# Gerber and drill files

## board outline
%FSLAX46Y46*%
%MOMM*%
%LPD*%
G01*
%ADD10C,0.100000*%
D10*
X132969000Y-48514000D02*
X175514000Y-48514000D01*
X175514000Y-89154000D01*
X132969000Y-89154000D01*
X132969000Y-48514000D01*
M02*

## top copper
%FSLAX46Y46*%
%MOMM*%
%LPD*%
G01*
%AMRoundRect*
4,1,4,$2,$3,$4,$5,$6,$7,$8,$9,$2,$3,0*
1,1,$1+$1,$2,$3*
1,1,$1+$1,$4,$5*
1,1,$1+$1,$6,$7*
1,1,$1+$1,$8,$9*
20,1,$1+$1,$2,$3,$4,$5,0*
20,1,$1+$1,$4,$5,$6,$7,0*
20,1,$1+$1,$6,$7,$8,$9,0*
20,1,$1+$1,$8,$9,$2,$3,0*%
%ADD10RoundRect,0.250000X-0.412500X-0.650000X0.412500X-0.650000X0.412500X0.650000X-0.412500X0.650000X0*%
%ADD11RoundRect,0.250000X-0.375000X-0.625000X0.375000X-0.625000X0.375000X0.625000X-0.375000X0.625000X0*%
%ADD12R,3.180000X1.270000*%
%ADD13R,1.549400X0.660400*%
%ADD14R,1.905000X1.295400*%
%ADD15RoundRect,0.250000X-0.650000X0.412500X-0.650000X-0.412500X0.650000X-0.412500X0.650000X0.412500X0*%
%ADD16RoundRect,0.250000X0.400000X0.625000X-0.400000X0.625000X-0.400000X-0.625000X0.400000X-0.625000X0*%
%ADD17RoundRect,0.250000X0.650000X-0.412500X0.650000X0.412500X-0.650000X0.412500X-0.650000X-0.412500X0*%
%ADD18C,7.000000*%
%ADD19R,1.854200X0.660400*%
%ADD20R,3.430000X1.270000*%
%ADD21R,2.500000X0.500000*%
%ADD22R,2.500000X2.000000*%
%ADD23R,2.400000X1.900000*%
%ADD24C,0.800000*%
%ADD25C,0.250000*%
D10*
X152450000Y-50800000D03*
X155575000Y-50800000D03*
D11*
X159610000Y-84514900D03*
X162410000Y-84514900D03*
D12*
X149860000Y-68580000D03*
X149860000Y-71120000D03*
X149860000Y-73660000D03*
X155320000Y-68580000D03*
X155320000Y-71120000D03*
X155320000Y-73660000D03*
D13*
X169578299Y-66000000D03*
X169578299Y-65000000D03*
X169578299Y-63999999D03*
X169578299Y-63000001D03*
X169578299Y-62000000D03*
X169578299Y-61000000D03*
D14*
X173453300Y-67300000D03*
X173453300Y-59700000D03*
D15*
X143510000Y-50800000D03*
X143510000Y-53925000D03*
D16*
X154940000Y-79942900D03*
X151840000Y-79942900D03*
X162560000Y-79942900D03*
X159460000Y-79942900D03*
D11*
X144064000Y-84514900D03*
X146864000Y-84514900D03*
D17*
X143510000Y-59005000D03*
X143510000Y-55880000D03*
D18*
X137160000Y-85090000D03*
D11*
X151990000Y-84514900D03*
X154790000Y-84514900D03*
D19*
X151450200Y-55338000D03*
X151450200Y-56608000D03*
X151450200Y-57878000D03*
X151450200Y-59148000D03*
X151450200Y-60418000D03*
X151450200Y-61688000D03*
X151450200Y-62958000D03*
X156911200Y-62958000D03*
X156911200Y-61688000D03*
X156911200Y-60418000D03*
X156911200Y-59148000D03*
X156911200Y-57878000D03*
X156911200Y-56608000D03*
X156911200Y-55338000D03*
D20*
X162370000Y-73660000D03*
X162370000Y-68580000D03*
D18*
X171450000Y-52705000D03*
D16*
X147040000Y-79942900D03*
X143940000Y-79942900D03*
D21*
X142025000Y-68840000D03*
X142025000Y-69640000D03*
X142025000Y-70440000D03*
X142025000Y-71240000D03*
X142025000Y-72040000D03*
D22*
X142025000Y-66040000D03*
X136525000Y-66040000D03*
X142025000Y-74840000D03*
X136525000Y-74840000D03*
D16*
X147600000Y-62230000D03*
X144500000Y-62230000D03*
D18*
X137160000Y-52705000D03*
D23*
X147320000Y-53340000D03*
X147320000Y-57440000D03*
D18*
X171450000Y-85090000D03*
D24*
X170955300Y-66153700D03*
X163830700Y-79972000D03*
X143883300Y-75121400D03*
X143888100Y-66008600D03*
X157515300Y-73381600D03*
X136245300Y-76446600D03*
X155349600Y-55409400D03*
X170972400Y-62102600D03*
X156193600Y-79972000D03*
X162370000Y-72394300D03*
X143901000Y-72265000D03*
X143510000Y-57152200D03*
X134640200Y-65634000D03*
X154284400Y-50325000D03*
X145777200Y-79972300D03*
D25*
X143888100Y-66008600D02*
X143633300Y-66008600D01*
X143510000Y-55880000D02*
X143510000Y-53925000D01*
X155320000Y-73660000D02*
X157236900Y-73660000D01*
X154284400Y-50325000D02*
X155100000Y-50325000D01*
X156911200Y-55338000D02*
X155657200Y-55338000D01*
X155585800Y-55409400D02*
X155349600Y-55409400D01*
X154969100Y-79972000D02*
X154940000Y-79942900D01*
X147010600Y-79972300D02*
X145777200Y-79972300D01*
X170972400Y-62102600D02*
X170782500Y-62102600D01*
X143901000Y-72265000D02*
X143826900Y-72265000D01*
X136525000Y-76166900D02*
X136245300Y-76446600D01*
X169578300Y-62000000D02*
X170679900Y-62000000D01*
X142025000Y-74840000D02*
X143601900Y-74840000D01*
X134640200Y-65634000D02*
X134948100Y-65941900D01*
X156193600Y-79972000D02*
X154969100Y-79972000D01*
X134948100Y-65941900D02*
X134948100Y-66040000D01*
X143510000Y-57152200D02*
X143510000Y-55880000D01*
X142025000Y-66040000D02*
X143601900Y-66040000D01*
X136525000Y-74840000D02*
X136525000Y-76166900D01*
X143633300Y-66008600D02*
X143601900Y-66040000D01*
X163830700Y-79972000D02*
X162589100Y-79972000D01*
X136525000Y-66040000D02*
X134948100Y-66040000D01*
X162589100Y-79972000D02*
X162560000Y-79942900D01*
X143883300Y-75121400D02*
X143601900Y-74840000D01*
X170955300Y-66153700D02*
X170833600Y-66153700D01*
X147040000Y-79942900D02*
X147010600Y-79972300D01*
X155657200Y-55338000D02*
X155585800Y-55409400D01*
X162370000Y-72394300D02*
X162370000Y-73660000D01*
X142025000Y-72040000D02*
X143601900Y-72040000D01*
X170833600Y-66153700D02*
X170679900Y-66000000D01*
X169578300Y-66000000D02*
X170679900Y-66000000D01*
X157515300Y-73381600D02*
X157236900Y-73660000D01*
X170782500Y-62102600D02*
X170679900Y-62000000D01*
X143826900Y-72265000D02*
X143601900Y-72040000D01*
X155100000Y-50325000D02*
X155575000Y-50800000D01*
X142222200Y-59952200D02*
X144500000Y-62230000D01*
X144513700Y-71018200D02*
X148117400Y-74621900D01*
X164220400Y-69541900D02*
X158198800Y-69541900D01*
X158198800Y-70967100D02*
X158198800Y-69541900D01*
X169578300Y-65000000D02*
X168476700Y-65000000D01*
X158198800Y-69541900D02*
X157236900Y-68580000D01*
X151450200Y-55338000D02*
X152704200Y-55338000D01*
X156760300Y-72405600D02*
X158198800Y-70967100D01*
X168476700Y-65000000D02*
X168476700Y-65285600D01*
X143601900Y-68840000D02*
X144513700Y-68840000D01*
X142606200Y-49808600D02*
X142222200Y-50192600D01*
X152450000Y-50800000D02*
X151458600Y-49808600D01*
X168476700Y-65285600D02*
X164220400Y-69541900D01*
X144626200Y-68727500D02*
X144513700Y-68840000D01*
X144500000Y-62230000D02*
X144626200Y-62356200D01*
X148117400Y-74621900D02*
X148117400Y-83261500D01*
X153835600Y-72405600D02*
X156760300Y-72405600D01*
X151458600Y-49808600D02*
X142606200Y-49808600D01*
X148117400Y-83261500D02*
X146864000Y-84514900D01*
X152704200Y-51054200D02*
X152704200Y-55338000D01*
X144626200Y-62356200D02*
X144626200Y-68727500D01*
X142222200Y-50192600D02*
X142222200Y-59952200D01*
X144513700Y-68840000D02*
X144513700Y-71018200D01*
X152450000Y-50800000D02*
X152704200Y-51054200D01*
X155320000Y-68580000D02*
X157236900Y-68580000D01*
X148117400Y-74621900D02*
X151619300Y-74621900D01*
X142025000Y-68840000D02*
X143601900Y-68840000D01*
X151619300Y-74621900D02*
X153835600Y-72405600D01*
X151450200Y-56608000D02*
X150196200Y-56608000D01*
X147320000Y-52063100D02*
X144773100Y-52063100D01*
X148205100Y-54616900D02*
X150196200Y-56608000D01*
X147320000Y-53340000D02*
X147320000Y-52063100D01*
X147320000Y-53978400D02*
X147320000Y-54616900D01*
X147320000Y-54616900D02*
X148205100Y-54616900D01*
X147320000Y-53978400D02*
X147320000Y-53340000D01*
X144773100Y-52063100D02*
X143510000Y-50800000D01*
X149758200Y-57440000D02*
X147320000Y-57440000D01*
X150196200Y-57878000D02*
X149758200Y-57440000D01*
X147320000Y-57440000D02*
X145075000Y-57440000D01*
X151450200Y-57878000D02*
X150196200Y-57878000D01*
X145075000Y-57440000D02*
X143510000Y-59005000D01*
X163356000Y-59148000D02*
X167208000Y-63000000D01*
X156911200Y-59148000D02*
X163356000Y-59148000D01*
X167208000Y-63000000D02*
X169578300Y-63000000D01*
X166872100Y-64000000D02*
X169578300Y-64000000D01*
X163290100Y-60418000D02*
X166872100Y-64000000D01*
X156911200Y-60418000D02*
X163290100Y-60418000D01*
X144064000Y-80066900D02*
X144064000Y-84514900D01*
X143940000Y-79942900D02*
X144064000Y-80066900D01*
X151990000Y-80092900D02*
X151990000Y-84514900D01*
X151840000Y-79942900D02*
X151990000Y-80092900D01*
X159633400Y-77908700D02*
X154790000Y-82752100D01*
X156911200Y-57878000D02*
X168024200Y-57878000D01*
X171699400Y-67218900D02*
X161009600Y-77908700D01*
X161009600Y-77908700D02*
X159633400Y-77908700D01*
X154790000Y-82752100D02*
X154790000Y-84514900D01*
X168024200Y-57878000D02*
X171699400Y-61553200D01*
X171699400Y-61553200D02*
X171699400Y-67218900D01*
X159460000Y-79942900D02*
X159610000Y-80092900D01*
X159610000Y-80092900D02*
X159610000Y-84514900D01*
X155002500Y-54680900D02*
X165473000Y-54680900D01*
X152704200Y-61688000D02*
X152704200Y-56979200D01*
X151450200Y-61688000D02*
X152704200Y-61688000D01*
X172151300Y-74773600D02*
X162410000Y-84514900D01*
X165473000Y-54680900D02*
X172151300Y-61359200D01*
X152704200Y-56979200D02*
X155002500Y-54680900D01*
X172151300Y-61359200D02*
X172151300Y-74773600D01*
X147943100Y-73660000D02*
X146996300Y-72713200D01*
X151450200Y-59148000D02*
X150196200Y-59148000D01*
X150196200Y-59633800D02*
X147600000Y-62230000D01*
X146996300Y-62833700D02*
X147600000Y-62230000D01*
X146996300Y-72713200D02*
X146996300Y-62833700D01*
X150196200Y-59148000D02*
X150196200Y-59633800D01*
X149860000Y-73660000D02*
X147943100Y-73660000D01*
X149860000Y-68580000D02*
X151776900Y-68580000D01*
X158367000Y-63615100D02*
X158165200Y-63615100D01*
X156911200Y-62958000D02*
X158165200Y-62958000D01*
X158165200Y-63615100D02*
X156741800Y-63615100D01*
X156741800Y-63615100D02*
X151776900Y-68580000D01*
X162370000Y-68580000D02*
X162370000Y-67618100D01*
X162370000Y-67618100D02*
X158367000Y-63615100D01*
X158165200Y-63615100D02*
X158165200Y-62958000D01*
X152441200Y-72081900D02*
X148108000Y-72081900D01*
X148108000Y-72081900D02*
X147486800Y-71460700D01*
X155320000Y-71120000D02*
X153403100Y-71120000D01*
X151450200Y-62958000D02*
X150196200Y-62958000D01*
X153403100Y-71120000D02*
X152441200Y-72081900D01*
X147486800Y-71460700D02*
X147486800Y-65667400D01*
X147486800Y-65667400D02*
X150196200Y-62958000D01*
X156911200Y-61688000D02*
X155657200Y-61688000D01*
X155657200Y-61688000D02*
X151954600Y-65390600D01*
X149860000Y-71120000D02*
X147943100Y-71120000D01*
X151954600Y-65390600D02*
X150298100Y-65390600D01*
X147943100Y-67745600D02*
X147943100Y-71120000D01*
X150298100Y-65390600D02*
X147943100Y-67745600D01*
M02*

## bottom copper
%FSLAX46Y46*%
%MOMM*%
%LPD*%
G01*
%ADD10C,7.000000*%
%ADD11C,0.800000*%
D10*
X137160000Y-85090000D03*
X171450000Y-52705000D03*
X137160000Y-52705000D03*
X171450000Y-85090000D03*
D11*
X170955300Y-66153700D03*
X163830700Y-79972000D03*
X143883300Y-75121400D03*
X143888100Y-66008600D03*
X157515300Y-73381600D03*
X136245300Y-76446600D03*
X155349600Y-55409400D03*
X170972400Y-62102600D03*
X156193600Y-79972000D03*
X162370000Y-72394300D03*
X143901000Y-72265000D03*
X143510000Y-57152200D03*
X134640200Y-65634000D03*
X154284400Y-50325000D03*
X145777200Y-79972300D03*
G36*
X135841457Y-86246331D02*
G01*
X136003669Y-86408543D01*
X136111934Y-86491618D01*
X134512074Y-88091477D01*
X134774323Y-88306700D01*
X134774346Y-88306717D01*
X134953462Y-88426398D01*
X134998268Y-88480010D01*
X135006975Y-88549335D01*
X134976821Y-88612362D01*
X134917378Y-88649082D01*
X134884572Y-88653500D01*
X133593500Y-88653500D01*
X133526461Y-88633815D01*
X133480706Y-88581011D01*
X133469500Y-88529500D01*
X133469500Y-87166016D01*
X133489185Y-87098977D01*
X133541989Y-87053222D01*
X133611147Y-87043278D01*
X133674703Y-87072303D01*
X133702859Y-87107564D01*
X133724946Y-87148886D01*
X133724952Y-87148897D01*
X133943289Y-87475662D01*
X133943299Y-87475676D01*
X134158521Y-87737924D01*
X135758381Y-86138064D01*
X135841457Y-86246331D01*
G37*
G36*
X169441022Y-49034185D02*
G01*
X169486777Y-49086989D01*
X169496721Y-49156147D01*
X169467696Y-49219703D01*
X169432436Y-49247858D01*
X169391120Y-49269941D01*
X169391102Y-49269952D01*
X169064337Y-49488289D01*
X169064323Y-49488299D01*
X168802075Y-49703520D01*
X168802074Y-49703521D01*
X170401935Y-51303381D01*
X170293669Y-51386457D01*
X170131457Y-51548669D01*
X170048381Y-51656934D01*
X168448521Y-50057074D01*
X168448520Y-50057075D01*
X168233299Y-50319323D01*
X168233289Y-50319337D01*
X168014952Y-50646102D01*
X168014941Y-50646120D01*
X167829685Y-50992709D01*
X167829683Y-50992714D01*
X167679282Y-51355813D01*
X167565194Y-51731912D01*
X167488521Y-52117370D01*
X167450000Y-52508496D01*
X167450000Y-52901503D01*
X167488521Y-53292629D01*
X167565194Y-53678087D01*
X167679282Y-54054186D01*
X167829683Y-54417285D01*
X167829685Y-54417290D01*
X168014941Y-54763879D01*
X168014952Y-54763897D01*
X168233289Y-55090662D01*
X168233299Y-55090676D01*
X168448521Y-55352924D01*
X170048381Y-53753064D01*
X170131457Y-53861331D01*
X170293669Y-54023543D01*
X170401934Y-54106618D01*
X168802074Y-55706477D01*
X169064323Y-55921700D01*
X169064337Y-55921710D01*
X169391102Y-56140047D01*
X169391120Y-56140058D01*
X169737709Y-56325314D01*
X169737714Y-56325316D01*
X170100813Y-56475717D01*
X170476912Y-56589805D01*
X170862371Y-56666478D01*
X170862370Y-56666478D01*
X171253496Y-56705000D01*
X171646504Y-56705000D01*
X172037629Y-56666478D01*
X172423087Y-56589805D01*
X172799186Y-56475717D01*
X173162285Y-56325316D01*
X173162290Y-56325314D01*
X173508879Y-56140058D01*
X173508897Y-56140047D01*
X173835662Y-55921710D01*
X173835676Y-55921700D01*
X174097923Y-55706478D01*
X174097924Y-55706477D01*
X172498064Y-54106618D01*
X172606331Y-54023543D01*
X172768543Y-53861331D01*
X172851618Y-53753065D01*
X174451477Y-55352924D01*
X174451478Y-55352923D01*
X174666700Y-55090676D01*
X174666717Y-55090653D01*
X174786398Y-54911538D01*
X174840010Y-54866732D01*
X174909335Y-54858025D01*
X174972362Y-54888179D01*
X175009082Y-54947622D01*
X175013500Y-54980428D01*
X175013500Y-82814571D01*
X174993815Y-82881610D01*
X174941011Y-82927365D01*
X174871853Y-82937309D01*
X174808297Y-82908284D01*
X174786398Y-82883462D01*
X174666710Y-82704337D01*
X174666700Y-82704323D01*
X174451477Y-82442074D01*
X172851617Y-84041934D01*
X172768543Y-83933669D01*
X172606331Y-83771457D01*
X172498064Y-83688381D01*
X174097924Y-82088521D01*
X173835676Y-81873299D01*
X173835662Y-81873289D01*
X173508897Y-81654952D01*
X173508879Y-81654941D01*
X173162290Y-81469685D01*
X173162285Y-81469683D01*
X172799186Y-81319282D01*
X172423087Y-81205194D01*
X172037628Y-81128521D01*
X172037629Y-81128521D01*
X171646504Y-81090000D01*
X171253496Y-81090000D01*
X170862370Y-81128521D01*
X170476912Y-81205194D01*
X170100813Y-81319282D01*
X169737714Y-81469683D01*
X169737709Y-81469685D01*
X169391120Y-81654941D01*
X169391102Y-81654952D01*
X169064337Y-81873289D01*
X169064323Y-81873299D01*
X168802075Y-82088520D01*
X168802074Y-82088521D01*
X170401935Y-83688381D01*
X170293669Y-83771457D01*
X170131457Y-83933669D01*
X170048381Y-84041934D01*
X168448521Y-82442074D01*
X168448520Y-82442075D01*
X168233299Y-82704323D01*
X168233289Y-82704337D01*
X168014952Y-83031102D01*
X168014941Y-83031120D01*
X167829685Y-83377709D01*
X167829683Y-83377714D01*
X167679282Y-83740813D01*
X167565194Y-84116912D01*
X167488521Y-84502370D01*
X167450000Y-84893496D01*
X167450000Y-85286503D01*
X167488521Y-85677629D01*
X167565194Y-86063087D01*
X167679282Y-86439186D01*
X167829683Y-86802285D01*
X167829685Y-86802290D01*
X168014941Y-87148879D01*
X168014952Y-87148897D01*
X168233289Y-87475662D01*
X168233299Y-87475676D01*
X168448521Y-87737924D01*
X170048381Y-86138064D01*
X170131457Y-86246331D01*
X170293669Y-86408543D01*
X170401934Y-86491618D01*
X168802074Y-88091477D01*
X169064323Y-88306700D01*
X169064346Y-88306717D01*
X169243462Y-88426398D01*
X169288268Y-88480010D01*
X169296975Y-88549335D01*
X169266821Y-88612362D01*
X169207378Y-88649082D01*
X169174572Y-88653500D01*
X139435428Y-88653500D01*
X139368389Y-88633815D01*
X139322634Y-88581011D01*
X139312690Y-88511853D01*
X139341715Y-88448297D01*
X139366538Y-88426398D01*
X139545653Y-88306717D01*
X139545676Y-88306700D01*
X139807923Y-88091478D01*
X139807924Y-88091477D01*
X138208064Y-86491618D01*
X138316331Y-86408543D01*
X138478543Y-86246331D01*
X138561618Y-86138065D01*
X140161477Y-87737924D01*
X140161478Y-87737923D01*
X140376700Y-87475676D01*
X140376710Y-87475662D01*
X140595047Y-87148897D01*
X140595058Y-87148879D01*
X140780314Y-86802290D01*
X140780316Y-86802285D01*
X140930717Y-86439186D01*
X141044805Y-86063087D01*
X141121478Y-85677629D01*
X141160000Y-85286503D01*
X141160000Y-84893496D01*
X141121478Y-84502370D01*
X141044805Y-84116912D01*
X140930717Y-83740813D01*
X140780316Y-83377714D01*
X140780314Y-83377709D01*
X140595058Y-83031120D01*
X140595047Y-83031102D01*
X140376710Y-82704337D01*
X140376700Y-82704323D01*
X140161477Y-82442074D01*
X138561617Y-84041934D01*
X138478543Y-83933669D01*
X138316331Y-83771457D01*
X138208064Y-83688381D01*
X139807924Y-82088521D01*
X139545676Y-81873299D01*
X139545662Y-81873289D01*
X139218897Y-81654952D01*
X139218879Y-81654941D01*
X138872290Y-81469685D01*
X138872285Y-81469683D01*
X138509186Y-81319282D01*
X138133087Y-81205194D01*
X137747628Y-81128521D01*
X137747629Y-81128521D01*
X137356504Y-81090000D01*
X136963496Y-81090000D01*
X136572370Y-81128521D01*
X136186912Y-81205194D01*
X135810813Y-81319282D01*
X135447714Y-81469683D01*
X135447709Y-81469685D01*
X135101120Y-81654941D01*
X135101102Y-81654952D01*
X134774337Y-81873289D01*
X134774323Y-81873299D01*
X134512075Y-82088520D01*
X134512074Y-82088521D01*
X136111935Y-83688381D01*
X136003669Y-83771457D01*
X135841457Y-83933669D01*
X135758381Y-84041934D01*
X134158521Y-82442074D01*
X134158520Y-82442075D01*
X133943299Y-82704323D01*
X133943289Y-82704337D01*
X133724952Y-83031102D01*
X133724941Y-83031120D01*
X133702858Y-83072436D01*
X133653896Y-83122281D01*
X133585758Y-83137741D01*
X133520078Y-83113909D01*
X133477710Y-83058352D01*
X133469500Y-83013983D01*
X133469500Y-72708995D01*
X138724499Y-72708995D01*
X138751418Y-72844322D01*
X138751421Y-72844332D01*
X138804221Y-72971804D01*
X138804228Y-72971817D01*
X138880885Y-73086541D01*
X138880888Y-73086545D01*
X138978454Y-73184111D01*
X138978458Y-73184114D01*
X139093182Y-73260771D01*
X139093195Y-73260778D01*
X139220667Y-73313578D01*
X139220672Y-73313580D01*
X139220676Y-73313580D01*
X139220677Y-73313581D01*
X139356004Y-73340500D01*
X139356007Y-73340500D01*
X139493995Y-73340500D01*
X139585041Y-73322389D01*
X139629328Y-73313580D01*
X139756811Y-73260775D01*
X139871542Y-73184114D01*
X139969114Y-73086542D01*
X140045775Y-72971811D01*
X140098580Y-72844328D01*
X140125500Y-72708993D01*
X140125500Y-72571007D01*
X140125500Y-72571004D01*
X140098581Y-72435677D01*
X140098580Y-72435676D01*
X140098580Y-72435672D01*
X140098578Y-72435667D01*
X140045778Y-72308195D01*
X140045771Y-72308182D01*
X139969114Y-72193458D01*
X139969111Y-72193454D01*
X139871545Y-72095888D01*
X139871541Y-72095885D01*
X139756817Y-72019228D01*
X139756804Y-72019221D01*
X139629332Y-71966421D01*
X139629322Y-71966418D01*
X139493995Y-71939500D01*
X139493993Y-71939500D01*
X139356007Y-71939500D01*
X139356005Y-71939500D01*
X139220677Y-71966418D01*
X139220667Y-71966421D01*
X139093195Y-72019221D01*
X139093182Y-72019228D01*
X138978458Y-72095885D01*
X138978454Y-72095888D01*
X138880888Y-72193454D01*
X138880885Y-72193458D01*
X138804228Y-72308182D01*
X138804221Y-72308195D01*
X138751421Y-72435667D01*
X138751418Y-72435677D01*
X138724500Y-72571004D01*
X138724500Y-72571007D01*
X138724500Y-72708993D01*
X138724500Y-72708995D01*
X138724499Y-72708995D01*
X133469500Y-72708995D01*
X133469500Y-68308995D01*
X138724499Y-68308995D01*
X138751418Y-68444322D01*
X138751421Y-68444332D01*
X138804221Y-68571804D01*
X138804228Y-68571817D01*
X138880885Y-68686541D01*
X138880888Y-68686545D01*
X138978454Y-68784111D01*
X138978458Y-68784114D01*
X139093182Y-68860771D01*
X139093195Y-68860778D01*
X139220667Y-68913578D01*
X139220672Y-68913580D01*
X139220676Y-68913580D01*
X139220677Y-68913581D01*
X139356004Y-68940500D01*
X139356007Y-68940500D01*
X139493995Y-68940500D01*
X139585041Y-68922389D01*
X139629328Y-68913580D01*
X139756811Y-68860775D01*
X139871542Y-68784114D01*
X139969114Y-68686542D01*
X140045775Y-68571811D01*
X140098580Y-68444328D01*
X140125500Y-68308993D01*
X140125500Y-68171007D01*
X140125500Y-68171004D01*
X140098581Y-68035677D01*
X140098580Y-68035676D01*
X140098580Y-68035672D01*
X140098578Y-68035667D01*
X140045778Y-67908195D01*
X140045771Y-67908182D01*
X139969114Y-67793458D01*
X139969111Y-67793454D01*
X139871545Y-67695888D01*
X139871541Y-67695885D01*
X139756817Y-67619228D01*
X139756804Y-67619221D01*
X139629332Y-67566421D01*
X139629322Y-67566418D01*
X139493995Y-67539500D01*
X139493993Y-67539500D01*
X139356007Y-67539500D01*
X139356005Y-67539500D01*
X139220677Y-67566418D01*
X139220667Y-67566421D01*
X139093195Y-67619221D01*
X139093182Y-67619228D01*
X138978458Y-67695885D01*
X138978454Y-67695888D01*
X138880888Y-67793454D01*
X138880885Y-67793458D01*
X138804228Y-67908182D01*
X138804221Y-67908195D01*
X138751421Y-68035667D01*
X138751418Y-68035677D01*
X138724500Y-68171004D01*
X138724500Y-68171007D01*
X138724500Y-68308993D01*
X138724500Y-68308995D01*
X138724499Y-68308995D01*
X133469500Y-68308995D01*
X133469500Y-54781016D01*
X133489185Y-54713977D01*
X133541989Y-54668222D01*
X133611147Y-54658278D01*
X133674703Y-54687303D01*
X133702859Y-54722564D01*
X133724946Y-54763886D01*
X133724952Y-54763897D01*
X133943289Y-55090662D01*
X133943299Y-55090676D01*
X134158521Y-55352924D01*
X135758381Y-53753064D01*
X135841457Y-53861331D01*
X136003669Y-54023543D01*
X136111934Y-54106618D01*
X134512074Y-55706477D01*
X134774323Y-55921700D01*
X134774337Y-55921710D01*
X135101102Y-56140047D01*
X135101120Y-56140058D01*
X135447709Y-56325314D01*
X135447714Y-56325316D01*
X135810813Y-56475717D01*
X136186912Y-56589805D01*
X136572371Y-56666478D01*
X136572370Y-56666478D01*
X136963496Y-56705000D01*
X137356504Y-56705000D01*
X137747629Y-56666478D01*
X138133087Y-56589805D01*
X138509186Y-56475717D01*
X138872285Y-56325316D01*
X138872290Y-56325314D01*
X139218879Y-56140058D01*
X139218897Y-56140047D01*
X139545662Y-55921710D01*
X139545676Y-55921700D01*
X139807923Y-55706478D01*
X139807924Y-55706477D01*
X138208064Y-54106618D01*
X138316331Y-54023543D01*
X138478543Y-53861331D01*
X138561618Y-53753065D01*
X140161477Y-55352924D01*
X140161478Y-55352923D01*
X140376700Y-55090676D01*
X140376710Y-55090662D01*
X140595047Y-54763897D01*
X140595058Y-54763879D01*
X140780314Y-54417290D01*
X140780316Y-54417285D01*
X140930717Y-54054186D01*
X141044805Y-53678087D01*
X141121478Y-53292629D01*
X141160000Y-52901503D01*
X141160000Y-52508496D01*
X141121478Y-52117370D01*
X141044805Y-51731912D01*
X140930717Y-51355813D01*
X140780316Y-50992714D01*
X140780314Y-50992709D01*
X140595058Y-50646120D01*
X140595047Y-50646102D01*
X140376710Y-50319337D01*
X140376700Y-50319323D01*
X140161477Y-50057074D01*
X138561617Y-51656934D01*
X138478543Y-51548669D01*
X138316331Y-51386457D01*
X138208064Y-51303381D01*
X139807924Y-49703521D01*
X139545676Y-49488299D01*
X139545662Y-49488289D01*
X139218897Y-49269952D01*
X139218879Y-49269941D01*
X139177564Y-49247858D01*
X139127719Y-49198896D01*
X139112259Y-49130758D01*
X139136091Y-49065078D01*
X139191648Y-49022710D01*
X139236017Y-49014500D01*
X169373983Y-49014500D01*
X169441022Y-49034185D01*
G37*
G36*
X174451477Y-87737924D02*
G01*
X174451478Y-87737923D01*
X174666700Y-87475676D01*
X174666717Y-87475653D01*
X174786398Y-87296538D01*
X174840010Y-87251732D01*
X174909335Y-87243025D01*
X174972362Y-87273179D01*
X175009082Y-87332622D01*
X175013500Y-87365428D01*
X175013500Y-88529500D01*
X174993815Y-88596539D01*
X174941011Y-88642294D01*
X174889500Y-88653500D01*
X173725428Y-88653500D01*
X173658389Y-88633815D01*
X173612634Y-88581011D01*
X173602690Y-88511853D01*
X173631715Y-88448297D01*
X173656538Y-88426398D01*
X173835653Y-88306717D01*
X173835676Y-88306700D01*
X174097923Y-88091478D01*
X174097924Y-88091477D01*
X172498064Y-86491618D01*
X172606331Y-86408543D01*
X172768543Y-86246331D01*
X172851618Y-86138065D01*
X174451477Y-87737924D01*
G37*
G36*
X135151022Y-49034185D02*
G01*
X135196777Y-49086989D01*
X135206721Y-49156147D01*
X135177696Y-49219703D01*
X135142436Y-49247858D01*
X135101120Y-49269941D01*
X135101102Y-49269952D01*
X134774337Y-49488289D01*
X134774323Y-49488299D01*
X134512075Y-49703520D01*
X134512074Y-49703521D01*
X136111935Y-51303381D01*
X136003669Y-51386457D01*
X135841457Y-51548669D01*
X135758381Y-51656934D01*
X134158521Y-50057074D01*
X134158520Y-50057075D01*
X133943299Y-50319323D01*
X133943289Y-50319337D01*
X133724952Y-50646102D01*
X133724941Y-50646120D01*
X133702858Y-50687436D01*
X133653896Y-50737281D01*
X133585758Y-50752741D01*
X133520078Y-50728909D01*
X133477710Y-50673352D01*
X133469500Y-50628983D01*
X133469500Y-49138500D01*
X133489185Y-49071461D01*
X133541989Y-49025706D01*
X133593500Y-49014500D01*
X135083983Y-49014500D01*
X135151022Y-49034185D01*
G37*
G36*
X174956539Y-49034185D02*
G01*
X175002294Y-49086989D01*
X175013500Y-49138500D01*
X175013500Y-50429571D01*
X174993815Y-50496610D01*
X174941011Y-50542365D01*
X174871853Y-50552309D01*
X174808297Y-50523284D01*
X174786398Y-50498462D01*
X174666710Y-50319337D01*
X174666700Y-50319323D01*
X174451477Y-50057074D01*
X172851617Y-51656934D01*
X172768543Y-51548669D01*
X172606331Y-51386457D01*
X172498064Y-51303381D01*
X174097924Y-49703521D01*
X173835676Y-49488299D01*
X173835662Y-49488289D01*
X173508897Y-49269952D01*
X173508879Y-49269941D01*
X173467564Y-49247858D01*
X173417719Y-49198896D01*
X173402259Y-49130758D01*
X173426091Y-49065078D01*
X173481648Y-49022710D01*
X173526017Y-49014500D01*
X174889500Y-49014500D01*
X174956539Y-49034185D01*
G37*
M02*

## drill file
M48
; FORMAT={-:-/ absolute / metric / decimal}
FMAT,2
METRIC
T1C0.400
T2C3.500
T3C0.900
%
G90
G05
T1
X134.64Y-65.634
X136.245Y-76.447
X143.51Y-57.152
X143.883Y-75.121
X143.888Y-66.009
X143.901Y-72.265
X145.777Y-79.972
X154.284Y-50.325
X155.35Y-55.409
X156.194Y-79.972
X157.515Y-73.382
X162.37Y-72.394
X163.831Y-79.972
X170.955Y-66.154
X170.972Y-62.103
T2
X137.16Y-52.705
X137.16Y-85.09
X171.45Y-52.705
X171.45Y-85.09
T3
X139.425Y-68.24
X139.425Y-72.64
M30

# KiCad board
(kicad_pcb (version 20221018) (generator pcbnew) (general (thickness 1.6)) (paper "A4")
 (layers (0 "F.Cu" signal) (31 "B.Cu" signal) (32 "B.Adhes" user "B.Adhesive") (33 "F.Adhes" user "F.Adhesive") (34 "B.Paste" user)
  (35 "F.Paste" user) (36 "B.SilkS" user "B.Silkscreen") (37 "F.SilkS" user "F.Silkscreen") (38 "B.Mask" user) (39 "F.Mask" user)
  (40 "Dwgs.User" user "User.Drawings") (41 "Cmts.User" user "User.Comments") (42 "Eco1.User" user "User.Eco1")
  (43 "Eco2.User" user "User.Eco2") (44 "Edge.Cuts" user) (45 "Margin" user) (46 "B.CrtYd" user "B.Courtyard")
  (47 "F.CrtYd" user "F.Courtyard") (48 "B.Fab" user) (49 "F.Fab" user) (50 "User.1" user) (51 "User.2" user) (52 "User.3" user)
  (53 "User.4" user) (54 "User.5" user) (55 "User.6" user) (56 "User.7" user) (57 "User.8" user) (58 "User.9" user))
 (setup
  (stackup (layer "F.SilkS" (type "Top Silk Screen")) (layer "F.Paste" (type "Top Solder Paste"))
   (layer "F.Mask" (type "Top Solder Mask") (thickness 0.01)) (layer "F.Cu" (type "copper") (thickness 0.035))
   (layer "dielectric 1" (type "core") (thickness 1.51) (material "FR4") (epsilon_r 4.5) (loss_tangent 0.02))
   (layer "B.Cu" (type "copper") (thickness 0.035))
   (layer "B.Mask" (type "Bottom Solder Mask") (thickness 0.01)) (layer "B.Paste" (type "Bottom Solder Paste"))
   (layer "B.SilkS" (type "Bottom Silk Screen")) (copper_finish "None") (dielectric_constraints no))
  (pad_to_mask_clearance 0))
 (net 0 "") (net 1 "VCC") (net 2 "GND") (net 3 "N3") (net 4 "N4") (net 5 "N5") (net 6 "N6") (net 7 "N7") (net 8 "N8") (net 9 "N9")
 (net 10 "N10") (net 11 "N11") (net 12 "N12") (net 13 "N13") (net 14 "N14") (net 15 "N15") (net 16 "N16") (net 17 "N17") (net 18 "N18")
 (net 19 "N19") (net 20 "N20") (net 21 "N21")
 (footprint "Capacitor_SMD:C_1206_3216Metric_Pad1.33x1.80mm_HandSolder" (layer "F.Cu") (at 154.0125 50.8)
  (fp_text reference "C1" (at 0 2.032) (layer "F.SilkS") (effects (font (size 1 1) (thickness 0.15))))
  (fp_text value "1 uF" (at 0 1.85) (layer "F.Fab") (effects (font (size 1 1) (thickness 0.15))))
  (pad "1" smd roundrect (at -1.5625 0) (size 1.325 1.8) (layers "F.Cu" "F.Paste" "F.Mask") (roundrect_rratio 0.188679) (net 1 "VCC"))
  (pad "2" smd roundrect (at 1.5625 0) (size 1.325 1.8) (layers "F.Cu" "F.Paste" "F.Mask") (roundrect_rratio 0.188679) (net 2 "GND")))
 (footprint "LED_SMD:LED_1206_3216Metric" (layer "F.Cu") (at 161.01 84.5149)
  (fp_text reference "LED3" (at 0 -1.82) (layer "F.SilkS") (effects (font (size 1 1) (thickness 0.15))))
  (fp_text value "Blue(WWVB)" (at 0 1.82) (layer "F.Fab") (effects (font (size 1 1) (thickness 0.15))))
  (pad "1" smd roundrect (at -1.4 0) (size 1.25 1.75) (layers "F.Cu" "F.Paste" "F.Mask") (roundrect_rratio 0.2) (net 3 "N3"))
  (pad "2" smd roundrect (at 1.4 0) (size 1.25 1.75) (layers "F.Cu" "F.Paste" "F.Mask") (roundrect_rratio 0.2) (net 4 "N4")))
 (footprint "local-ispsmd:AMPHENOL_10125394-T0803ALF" (layer "F.Cu") (at 152.59 71.12 -90)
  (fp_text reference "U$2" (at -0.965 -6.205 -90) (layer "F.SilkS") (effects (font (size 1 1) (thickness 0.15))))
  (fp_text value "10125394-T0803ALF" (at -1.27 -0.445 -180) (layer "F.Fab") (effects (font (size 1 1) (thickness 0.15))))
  (pad "A01" smd rect (at -2.54 2.73 270) (size 1.27 3.18) (layers "F.Cu" "F.Paste" "F.Mask") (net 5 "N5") (solder_mask_margin 0.102))
  (pad "A02" smd rect (at 0 2.73 270) (size 1.27 3.18) (layers "F.Cu" "F.Paste" "F.Mask") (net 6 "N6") (solder_mask_margin 0.102))
  (pad "A03" smd rect (at 2.54 2.73 270) (size 1.27 3.18) (layers "F.Cu" "F.Paste" "F.Mask") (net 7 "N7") (solder_mask_margin 0.102))
  (pad "B01" smd rect (at -2.54 -2.73 270) (size 1.27 3.18) (layers "F.Cu" "F.Paste" "F.Mask") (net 1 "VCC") (solder_mask_margin 0.102))
  (pad "B02" smd rect (at 0 -2.73 270) (size 1.27 3.18) (layers "F.Cu" "F.Paste" "F.Mask") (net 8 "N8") (solder_mask_margin 0.102))
  (pad "B03" smd rect (at 2.54 -2.73 270) (size 1.27 3.18) (layers "F.Cu" "F.Paste" "F.Mask") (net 2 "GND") (solder_mask_margin 0.102)))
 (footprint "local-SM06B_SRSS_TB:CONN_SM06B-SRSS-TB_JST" (layer "F.Cu") (at 172.085 63.5 90)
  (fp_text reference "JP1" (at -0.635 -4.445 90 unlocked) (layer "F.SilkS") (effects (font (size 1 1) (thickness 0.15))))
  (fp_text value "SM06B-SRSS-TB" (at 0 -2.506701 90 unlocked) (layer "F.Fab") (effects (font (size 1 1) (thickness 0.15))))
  (pad "1" smd rect (at -2.5 -2.506701 90) (size 0.6604 1.5494) (layers "F.Cu" "F.Paste" "F.Mask") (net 2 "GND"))
  (pad "2" smd rect (at -1.5 -2.506701 90) (size 0.6604 1.5494) (layers "F.Cu" "F.Paste" "F.Mask") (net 1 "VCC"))
  (pad "3" smd rect (at -0.499999 -2.506701 90) (size 0.6604 1.5494) (layers "F.Cu" "F.Paste" "F.Mask") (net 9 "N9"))
  (pad "4" smd rect (at 0.499999 -2.506701 90) (size 0.6604 1.5494) (layers "F.Cu" "F.Paste" "F.Mask") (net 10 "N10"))
  (pad "5" smd rect (at 1.5 -2.506701 90) (size 0.6604 1.5494) (layers "F.Cu" "F.Paste" "F.Mask") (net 2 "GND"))
  (pad "6" smd rect (at 2.5 -2.506701 90) (size 0.6604 1.5494) (layers "F.Cu" "F.Paste" "F.Mask") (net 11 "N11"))
  (pad "7" smd rect (at -3.8 1.3683 180) (size 1.905 1.2954) (layers "F.Cu" "F.Paste" "F.Mask"))
  (pad "8" smd rect (at 3.8 1.3683 180) (size 1.905 1.2954) (layers "F.Cu" "F.Paste" "F.Mask")))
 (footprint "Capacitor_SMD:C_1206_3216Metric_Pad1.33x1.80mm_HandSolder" (layer "F.Cu") (at 143.51 52.3625 -90)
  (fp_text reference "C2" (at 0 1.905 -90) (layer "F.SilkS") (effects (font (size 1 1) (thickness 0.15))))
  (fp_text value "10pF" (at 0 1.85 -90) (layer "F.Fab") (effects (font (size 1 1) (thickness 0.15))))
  (pad "1" smd roundrect (at -1.5625 0 270) (size 1.325 1.8) (layers "F.Cu" "F.Paste" "F.Mask") (roundrect_rratio 0.188679) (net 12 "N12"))
  (pad "2" smd roundrect (at 1.5625 0 270) (size 1.325 1.8) (layers "F.Cu" "F.Paste" "F.Mask") (roundrect_rratio 0.188679) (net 2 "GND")))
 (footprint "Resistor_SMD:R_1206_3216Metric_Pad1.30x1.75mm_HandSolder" (layer "F.Cu") (at 153.39 79.9429 180)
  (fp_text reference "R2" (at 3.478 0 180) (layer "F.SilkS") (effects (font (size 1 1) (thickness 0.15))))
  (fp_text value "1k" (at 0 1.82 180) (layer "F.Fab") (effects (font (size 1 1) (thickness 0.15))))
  (pad "1" smd roundrect (at -1.55 0 180) (size 1.3 1.75) (layers "F.Cu" "F.Paste" "F.Mask") (roundrect_rratio 0.192308) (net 2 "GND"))
  (pad "2" smd roundrect (at 1.55 0 180) (size 1.3 1.75) (layers "F.Cu" "F.Paste" "F.Mask") (roundrect_rratio 0.192308) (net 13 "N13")))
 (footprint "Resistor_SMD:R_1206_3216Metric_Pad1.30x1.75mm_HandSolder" (layer "F.Cu") (at 161.01 79.9429 180)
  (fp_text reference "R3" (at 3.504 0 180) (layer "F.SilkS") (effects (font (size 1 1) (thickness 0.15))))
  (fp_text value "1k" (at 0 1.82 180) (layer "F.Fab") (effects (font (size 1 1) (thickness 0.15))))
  (pad "1" smd roundrect (at -1.55 0 180) (size 1.3 1.75) (layers "F.Cu" "F.Paste" "F.Mask") (roundrect_rratio 0.192308) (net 2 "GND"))
  (pad "2" smd roundrect (at 1.55 0 180) (size 1.3 1.75) (layers "F.Cu" "F.Paste" "F.Mask") (roundrect_rratio 0.192308) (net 3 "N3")))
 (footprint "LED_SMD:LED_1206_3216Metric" (layer "F.Cu") (at 145.464 84.5149)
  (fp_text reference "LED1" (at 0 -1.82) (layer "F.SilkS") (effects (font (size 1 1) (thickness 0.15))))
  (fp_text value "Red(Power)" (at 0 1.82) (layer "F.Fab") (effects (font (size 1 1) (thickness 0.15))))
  (pad "1" smd roundrect (at -1.4 0) (size 1.25 1.75) (layers "F.Cu" "F.Paste" "F.Mask") (roundrect_rratio 0.2) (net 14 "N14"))
  (pad "2" smd roundrect (at 1.4 0) (size 1.25 1.75) (layers "F.Cu" "F.Paste" "F.Mask") (roundrect_rratio 0.2) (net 1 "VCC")))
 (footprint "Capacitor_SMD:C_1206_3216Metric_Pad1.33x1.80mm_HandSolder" (layer "F.Cu") (at 143.51 57.4425 90)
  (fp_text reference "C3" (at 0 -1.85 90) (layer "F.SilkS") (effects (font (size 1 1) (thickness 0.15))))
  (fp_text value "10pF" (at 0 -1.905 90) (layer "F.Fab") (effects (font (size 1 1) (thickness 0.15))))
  (pad "1" smd roundrect (at -1.5625 0 90) (size 1.325 1.8) (layers "F.Cu" "F.Paste" "F.Mask") (roundrect_rratio 0.188679) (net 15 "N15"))
  (pad "2" smd roundrect (at 1.5625 0 90) (size 1.325 1.8) (layers "F.Cu" "F.Paste" "F.Mask") (roundrect_rratio 0.188679) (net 2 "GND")))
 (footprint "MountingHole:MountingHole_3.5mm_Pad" (layer "F.Cu") (at 137.16 85.09)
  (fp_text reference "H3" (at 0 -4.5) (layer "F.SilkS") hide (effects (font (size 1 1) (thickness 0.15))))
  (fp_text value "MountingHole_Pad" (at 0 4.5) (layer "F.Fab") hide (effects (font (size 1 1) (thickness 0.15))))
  (pad "1" thru_hole circle (at 0 0) (size 7 7) (drill 3.5) (layers "*.Cu" "*.Mask") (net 2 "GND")))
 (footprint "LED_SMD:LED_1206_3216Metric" (layer "F.Cu") (at 153.39 84.5149)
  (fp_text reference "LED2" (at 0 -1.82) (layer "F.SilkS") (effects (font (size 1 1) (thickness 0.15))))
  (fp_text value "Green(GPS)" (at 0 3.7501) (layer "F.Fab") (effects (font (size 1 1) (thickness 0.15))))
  (pad "1" smd roundrect (at -1.4 0) (size 1.25 1.75) (layers "F.Cu" "F.Paste" "F.Mask") (roundrect_rratio 0.2) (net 13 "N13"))
  (pad "2" smd roundrect (at 1.4 0) (size 1.25 1.75) (layers "F.Cu" "F.Paste" "F.Mask") (roundrect_rratio 0.2) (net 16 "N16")))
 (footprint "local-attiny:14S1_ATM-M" (layer "F.Cu") (at 154.1807 59.148)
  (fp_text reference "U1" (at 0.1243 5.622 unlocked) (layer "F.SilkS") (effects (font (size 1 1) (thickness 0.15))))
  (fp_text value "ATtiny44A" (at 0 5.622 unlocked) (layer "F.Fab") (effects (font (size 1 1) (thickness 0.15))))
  (pad "1" smd rect (at -2.7305 -3.81) (size 1.8542 0.6604) (layers "F.Cu" "F.Paste" "F.Mask") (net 1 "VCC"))
  (pad "2" smd rect (at -2.7305 -2.54) (size 1.8542 0.6604) (layers "F.Cu" "F.Paste" "F.Mask") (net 12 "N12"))
  (pad "3" smd rect (at -2.7305 -1.27) (size 1.8542 0.6604) (layers "F.Cu" "F.Paste" "F.Mask") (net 15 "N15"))
  (pad "4" smd rect (at -2.7305 0) (size 1.8542 0.6604) (layers "F.Cu" "F.Paste" "F.Mask") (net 7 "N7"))
  (pad "5" smd rect (at -2.7305 1.27) (size 1.8542 0.6604) (layers "F.Cu" "F.Paste" "F.Mask") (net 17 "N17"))
  (pad "6" smd rect (at -2.7305 2.54) (size 1.8542 0.6604) (layers "F.Cu" "F.Paste" "F.Mask") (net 4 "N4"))
  (pad "7" smd rect (at -2.7305 3.81) (size 1.8542 0.6604) (layers "F.Cu" "F.Paste" "F.Mask") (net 8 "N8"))
  (pad "8" smd rect (at 2.7305 3.81) (size 1.8542 0.6604) (layers "F.Cu" "F.Paste" "F.Mask") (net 5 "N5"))
  (pad "9" smd rect (at 2.7305 2.54) (size 1.8542 0.6604) (layers "F.Cu" "F.Paste" "F.Mask") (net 6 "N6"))
  (pad "10" smd rect (at 2.7305 1.27) (size 1.8542 0.6604) (layers "F.Cu" "F.Paste" "F.Mask") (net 9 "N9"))
  (pad "11" smd rect (at 2.7305 0) (size 1.8542 0.6604) (layers "F.Cu" "F.Paste" "F.Mask") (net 10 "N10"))
  (pad "12" smd rect (at 2.7305 -1.27) (size 1.8542 0.6604) (layers "F.Cu" "F.Paste" "F.Mask") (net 16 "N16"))
  (pad "13" smd rect (at 2.7305 -2.54) (size 1.8542 0.6604) (layers "F.Cu" "F.Paste" "F.Mask") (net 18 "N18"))
  (pad "14" smd rect (at 2.7305 -3.81) (size 1.8542 0.6604) (layers "F.Cu" "F.Paste" "F.Mask") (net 2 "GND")))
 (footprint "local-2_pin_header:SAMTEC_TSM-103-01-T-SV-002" (layer "F.Cu") (at 163.83 71.12 -90)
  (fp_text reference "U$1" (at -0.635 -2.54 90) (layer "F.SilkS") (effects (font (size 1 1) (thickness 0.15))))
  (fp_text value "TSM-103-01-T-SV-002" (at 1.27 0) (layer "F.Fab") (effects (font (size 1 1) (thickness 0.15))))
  (pad "01" smd rect (at 2.54 1.46 270) (size 1.27 3.43) (layers "F.Cu" "F.Paste" "F.Mask") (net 2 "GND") (solder_mask_margin 0.102))
  (pad "03" smd rect (at -2.54 1.46 270) (size 1.27 3.43) (layers "F.Cu" "F.Paste" "F.Mask") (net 5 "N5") (solder_mask_margin 0.102)))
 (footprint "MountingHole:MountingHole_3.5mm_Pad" (layer "F.Cu") (at 171.45 52.705)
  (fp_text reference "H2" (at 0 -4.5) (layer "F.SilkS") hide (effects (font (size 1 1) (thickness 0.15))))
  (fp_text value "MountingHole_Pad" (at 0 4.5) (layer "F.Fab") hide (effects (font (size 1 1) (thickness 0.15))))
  (pad "1" thru_hole circle (at 0 0) (size 7 7) (drill 3.5) (layers "*.Cu" "*.Mask") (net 2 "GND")))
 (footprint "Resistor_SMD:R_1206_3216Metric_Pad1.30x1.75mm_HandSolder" (layer "F.Cu") (at 145.49 79.9429 180)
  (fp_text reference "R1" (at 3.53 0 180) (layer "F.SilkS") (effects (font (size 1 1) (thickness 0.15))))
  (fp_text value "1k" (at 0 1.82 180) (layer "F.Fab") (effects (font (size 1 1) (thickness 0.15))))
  (pad "1" smd roundrect (at -1.55 0 180) (size 1.3 1.75) (layers "F.Cu" "F.Paste" "F.Mask") (roundrect_rratio 0.192308) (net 2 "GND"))
  (pad "2" smd roundrect (at 1.55 0 180) (size 1.3 1.75) (layers "F.Cu" "F.Paste" "F.Mask") (roundrect_rratio 0.192308) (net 14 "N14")))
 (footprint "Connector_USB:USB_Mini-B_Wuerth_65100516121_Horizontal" (layer "F.Cu") (at 139.425 70.44 -90)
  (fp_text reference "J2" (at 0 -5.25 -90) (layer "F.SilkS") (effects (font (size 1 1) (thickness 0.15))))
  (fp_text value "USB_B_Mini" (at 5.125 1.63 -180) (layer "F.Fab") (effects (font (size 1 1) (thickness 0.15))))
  (pad "" np_thru_hole circle (at -2.2 0 270) (size 0.9 0.9) (drill 0.9) (layers "*.Cu" "*.Mask"))
  (pad "" np_thru_hole circle (at 2.2 0 270) (size 0.9 0.9) (drill 0.9) (layers "*.Cu" "*.Mask"))
  (pad "1" smd rect (at -1.6 -2.6 270) (size 0.5 2.5) (layers "F.Cu" "F.Paste" "F.Mask") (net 1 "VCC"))
  (pad "2" smd rect (at -0.8 -2.6 270) (size 0.5 2.5) (layers "F.Cu" "F.Paste" "F.Mask") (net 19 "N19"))
  (pad "3" smd rect (at 0 -2.6 270) (size 0.5 2.5) (layers "F.Cu" "F.Paste" "F.Mask") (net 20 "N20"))
  (pad "4" smd rect (at 0.8 -2.6 270) (size 0.5 2.5) (layers "F.Cu" "F.Paste" "F.Mask") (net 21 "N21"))
  (pad "5" smd rect (at 1.6 -2.6 270) (size 0.5 2.5) (layers "F.Cu" "F.Paste" "F.Mask") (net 2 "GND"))
  (pad "6" smd rect (at -4.4 -2.6 270) (size 2 2.5) (layers "F.Cu" "F.Paste" "F.Mask") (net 2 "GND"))
  (pad "6" smd rect (at -4.4 2.9 270) (size 2 2.5) (layers "F.Cu" "F.Paste" "F.Mask") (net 2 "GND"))
  (pad "6" smd rect (at 4.4 -2.6 270) (size 2 2.5) (layers "F.Cu" "F.Paste" "F.Mask") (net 2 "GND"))
  (pad "6" smd rect (at 4.4 2.9 270) (size 2 2.5) (layers "F.Cu" "F.Paste" "F.Mask") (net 2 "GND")))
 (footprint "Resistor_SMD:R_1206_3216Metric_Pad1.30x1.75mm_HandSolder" (layer "F.Cu") (at 146.05 62.23 180)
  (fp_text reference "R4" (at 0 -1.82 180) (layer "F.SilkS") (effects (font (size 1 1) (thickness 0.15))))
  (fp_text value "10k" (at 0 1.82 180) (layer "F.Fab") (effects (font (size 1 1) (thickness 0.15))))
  (pad "1" smd roundrect (at -1.55 0 180) (size 1.3 1.75) (layers "F.Cu" "F.Paste" "F.Mask") (roundrect_rratio 0.192308) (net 7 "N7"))
  (pad "2" smd roundrect (at 1.55 0 180) (size 1.3 1.75) (layers "F.Cu" "F.Paste" "F.Mask") (roundrect_rratio 0.192308) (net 1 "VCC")))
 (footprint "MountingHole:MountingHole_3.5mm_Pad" (layer "F.Cu") (at 137.16 52.705)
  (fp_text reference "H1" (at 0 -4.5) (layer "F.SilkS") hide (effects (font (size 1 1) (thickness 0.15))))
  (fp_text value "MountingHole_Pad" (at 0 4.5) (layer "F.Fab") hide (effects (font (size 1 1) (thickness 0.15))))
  (pad "1" thru_hole circle (at 0 0) (size 7 7) (drill 3.5) (layers "*.Cu" "*.Mask") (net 2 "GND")))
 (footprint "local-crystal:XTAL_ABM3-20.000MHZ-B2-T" (layer "F.Cu") (at 147.32 55.39 -90)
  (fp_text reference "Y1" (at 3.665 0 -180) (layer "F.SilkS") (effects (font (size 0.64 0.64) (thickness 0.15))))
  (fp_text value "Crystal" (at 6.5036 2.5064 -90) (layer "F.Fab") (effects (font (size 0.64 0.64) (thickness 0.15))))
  (pad "1" smd rect (at -2.05 0 270) (size 1.9 2.4) (layers "F.Cu" "F.Paste" "F.Mask") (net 12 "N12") (solder_mask_margin 0.102))
  (pad "2" smd rect (at 2.05 0 270) (size 1.9 2.4) (layers "F.Cu" "F.Paste" "F.Mask") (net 15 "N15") (solder_mask_margin 0.102)))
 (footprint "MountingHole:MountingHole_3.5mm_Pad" (layer "F.Cu") (at 171.45 85.09)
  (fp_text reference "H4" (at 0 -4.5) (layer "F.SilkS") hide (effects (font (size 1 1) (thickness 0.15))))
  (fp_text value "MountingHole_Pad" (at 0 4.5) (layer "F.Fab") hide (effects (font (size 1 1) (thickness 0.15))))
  (pad "1" thru_hole circle (at 0 0) (size 7 7) (drill 3.5) (layers "*.Cu" "*.Mask") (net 2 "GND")))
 (gr_rect (start 132.969 48.514) (end 175.514 89.154) (stroke (width 0.1) (type default)) (fill none) (layer "Edge.Cuts"))
 (segment (start 143.8881 66.0086) (end 143.6333 66.0086) (width 0.25) (layer "F.Cu") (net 2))
 (segment (start 143.51 55.88) (end 143.51 53.925) (width 0.25) (layer "F.Cu") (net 2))
 (segment (start 155.32 73.66) (end 157.2369 73.66) (width 0.25) (layer "F.Cu") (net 2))
 (segment (start 154.2844 50.325) (end 155.1 50.325) (width 0.25) (layer "F.Cu") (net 2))
 (segment (start 156.9112 55.338) (end 155.6572 55.338) (width 0.25) (layer "F.Cu") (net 2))
 (segment (start 155.5858 55.4094) (end 155.3496 55.4094) (width 0.25) (layer "F.Cu") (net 2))
 (segment (start 154.9691 79.972) (end 154.94 79.9429) (width 0.25) (layer "F.Cu") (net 2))
 (segment (start 147.0106 79.9723) (end 145.7772 79.9723) (width 0.25) (layer "F.Cu") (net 2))
 (segment (start 170.9724 62.1026) (end 170.7825 62.1026) (width 0.25) (layer "F.Cu") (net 2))
 (segment (start 143.901 72.265) (end 143.8269 72.265) (width 0.25) (layer "F.Cu") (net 2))
 (segment (start 136.525 76.1669) (end 136.2453 76.4466) (width 0.25) (layer "F.Cu") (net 2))
 (segment (start 169.5783 62) (end 170.6799 62) (width 0.25) (layer "F.Cu") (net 2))
 (segment (start 142.025 74.84) (end 143.6019 74.84) (width 0.25) (layer "F.Cu") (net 2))
 (segment (start 134.6402 65.634) (end 134.9481 65.9419) (width 0.25) (layer "F.Cu") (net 2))
 (segment (start 156.1936 79.972) (end 154.9691 79.972) (width 0.25) (layer "F.Cu") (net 2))
 (segment (start 134.9481 65.9419) (end 134.9481 66.04) (width 0.25) (layer "F.Cu") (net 2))
 (segment (start 143.51 57.1522) (end 143.51 55.88) (width 0.25) (layer "F.Cu") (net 2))
 (segment (start 142.025 66.04) (end 143.6019 66.04) (width 0.25) (layer "F.Cu") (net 2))
 (segment (start 136.525 74.84) (end 136.525 76.1669) (width 0.25) (layer "F.Cu") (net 2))
 (segment (start 143.6333 66.0086) (end 143.6019 66.04) (width 0.25) (layer "F.Cu") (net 2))
 (segment (start 163.8307 79.972) (end 162.5891 79.972) (width 0.25) (layer "F.Cu") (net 2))
 (segment (start 136.525 66.04) (end 134.9481 66.04) (width 0.25) (layer "F.Cu") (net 2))
 (segment (start 162.5891 79.972) (end 162.56 79.9429) (width 0.25) (layer "F.Cu") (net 2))
 (segment (start 143.8833 75.1214) (end 143.6019 74.84) (width 0.25) (layer "F.Cu") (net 2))
 (segment (start 170.9553 66.1537) (end 170.8336 66.1537) (width 0.25) (layer "F.Cu") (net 2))
 (segment (start 147.04 79.9429) (end 147.0106 79.9723) (width 0.25) (layer "F.Cu") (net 2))
 (segment (start 155.6572 55.338) (end 155.5858 55.4094) (width 0.25) (layer "F.Cu") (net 2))
 (segment (start 162.37 72.3943) (end 162.37 73.66) (width 0.25) (layer "F.Cu") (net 2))
 (segment (start 142.025 72.04) (end 143.6019 72.04) (width 0.25) (layer "F.Cu") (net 2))
 (segment (start 170.8336 66.1537) (end 170.6799 66) (width 0.25) (layer "F.Cu") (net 2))
 (segment (start 169.5783 66) (end 170.6799 66) (width 0.25) (layer "F.Cu") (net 2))
 (segment (start 157.5153 73.3816) (end 157.2369 73.66) (width 0.25) (layer "F.Cu") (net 2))
 (segment (start 170.7825 62.1026) (end 170.6799 62) (width 0.25) (layer "F.Cu") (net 2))
 (segment (start 143.8269 72.265) (end 143.6019 72.04) (width 0.25) (layer "F.Cu") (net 2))
 (segment (start 155.1 50.325) (end 155.575 50.8) (width 0.25) (layer "F.Cu") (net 2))
 (via (at 170.9553 66.1537) (size 0.8) (drill 0.4) (layers "F.Cu" "B.Cu") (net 2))
 (via (at 163.8307 79.972) (size 0.8) (drill 0.4) (layers "F.Cu" "B.Cu") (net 2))
 (via (at 143.8833 75.1214) (size 0.8) (drill 0.4) (layers "F.Cu" "B.Cu") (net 2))
 (via (at 143.8881 66.0086) (size 0.8) (drill 0.4) (layers "F.Cu" "B.Cu") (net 2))
 (via (at 157.5153 73.3816) (size 0.8) (drill 0.4) (layers "F.Cu" "B.Cu") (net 2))
 (via (at 136.2453 76.4466) (size 0.8) (drill 0.4) (layers "F.Cu" "B.Cu") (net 2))
 (via (at 155.3496 55.4094) (size 0.8) (drill 0.4) (layers "F.Cu" "B.Cu") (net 2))
 (via (at 170.9724 62.1026) (size 0.8) (drill 0.4) (layers "F.Cu" "B.Cu") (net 2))
 (via (at 156.1936 79.972) (size 0.8) (drill 0.4) (layers "F.Cu" "B.Cu") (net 2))
 (via (at 162.37 72.3943) (size 0.8) (drill 0.4) (layers "F.Cu" "B.Cu") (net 2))
 (via (at 143.901 72.265) (size 0.8) (drill 0.4) (layers "F.Cu" "B.Cu") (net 2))
 (via (at 143.51 57.1522) (size 0.8) (drill 0.4) (layers "F.Cu" "B.Cu") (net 2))
 (via (at 134.6402 65.634) (size 0.8) (drill 0.4) (layers "F.Cu" "B.Cu") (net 2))
 (via (at 154.2844 50.325) (size 0.8) (drill 0.4) (layers "F.Cu" "B.Cu") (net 2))
 (via (at 145.7772 79.9723) (size 0.8) (drill 0.4) (layers "F.Cu" "B.Cu") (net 2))
 (segment (start 142.2222 59.9522) (end 144.5 62.23) (width 0.25) (layer "F.Cu") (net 1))
 (segment (start 144.5137 71.0182) (end 148.1174 74.6219) (width 0.25) (layer "F.Cu") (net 1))
 (segment (start 164.2204 69.5419) (end 158.1988 69.5419) (width 0.25) (layer "F.Cu") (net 1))
 (segment (start 158.1988 70.9671) (end 158.1988 69.5419) (width 0.25) (layer "F.Cu") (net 1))
 (segment (start 169.5783 65) (end 168.4767 65) (width 0.25) (layer "F.Cu") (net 1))
 (segment (start 158.1988 69.5419) (end 157.2369 68.58) (width 0.25) (layer "F.Cu") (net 1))
 (segment (start 151.4502 55.338) (end 152.7042 55.338) (width 0.25) (layer "F.Cu") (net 1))
 (segment (start 156.7603 72.4056) (end 158.1988 70.9671) (width 0.25) (layer "F.Cu") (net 1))
 (segment (start 168.4767 65) (end 168.4767 65.2856) (width 0.25) (layer "F.Cu") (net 1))
 (segment (start 143.6019 68.84) (end 144.5137 68.84) (width 0.25) (layer "F.Cu") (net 1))
 (segment (start 142.6062 49.8086) (end 142.2222 50.1926) (width 0.25) (layer "F.Cu") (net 1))
 (segment (start 152.45 50.8) (end 151.4586 49.8086) (width 0.25) (layer "F.Cu") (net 1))
 (segment (start 168.4767 65.2856) (end 164.2204 69.5419) (width 0.25) (layer "F.Cu") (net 1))
 (segment (start 144.6262 68.7275) (end 144.5137 68.84) (width 0.25) (layer "F.Cu") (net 1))
 (segment (start 144.5 62.23) (end 144.6262 62.3562) (width 0.25) (layer "F.Cu") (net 1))
 (segment (start 148.1174 74.6219) (end 148.1174 83.2615) (width 0.25) (layer "F.Cu") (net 1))
 (segment (start 153.8356 72.4056) (end 156.7603 72.4056) (width 0.25) (layer "F.Cu") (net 1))
 (segment (start 151.4586 49.8086) (end 142.6062 49.8086) (width 0.25) (layer "F.Cu") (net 1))
 (segment (start 148.1174 83.2615) (end 146.864 84.5149) (width 0.25) (layer "F.Cu") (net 1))
 (segment (start 152.7042 51.0542) (end 152.7042 55.338) (width 0.25) (layer "F.Cu") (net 1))
 (segment (start 144.6262 62.3562) (end 144.6262 68.7275) (width 0.25) (layer "F.Cu") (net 1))
 (segment (start 142.2222 50.1926) (end 142.2222 59.9522) (width 0.25) (layer "F.Cu") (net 1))
 (segment (start 144.5137 68.84) (end 144.5137 71.0182) (width 0.25) (layer "F.Cu") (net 1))
 (segment (start 152.45 50.8) (end 152.7042 51.0542) (width 0.25) (layer "F.Cu") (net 1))
 (segment (start 155.32 68.58) (end 157.2369 68.58) (width 0.25) (layer "F.Cu") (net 1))
 (segment (start 148.1174 74.6219) (end 151.6193 74.6219) (width 0.25) (layer "F.Cu") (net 1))
 (segment (start 142.025 68.84) (end 143.6019 68.84) (width 0.25) (layer "F.Cu") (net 1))
 (segment (start 151.6193 74.6219) (end 153.8356 72.4056) (width 0.25) (layer "F.Cu") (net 1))
 (segment (start 151.4502 56.608) (end 150.1962 56.608) (width 0.25) (layer "F.Cu") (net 12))
 (segment (start 147.32 52.0631) (end 144.7731 52.0631) (width 0.25) (layer "F.Cu") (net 12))
 (segment (start 148.2051 54.6169) (end 150.1962 56.608) (width 0.25) (layer "F.Cu") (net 12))
 (segment (start 147.32 53.34) (end 147.32 52.0631) (width 0.25) (layer "F.Cu") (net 12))
 (segment (start 147.32 53.9784) (end 147.32 54.6169) (width 0.25) (layer "F.Cu") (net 12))
 (segment (start 147.32 54.6169) (end 148.2051 54.6169) (width 0.25) (layer "F.Cu") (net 12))
 (segment (start 147.32 53.9784) (end 147.32 53.34) (width 0.25) (layer "F.Cu") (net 12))
 (segment (start 144.7731 52.0631) (end 143.51 50.8) (width 0.25) (layer "F.Cu") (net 12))
 (segment (start 149.7582 57.44) (end 147.32 57.44) (width 0.25) (layer "F.Cu") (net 15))
 (segment (start 150.1962 57.878) (end 149.7582 57.44) (width 0.25) (layer "F.Cu") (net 15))
 (segment (start 147.32 57.44) (end 145.075 57.44) (width 0.25) (layer "F.Cu") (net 15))
 (segment (start 151.4502 57.878) (end 150.1962 57.878) (width 0.25) (layer "F.Cu") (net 15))
 (segment (start 145.075 57.44) (end 143.51 59.005) (width 0.25) (layer "F.Cu") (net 15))
 (segment (start 163.356 59.148) (end 167.208 63) (width 0.25) (layer "F.Cu") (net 10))
 (segment (start 156.9112 59.148) (end 163.356 59.148) (width 0.25) (layer "F.Cu") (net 10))
 (segment (start 167.208 63) (end 169.5783 63) (width 0.25) (layer "F.Cu") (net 10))
 (segment (start 166.8721 64) (end 169.5783 64) (width 0.25) (layer "F.Cu") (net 9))
 (segment (start 163.2901 60.418) (end 166.8721 64) (width 0.25) (layer "F.Cu") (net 9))
 (segment (start 156.9112 60.418) (end 163.2901 60.418) (width 0.25) (layer "F.Cu") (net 9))
 (segment (start 144.064 80.0669) (end 144.064 84.5149) (width 0.25) (layer "F.Cu") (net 14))
 (segment (start 143.94 79.9429) (end 144.064 80.0669) (width 0.25) (layer "F.Cu") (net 14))
 (segment (start 151.99 80.0929) (end 151.99 84.5149) (width 0.25) (layer "F.Cu") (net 13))
 (segment (start 151.84 79.9429) (end 151.99 80.0929) (width 0.25) (layer "F.Cu") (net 13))
 (segment (start 159.6334 77.9087) (end 154.79 82.7521) (width 0.25) (layer "F.Cu") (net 16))
 (segment (start 156.9112 57.878) (end 168.0242 57.878) (width 0.25) (layer "F.Cu") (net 16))
 (segment (start 171.6994 67.2189) (end 161.0096 77.9087) (width 0.25) (layer "F.Cu") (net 16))
 (segment (start 161.0096 77.9087) (end 159.6334 77.9087) (width 0.25) (layer "F.Cu") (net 16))
 (segment (start 154.79 82.7521) (end 154.79 84.5149) (width 0.25) (layer "F.Cu") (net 16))
 (segment (start 168.0242 57.878) (end 171.6994 61.5532) (width 0.25) (layer "F.Cu") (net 16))
 (segment (start 171.6994 61.5532) (end 171.6994 67.2189) (width 0.25) (layer "F.Cu") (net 16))
 (segment (start 159.46 79.9429) (end 159.61 80.0929) (width 0.25) (layer "F.Cu") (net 3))
 (segment (start 159.61 80.0929) (end 159.61 84.5149) (width 0.25) (layer "F.Cu") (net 3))
 (segment (start 155.0025 54.6809) (end 165.473 54.6809) (width 0.25) (layer "F.Cu") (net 4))
 (segment (start 152.7042 61.688) (end 152.7042 56.9792) (width 0.25) (layer "F.Cu") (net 4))
 (segment (start 151.4502 61.688) (end 152.7042 61.688) (width 0.25) (layer "F.Cu") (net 4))
 (segment (start 172.1513 74.7736) (end 162.41 84.5149) (width 0.25) (layer "F.Cu") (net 4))
 (segment (start 165.473 54.6809) (end 172.1513 61.3592) (width 0.25) (layer "F.Cu") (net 4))
 (segment (start 152.7042 56.9792) (end 155.0025 54.6809) (width 0.25) (layer "F.Cu") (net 4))
 (segment (start 172.1513 61.3592) (end 172.1513 74.7736) (width 0.25) (layer "F.Cu") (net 4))
 (segment (start 147.9431 73.66) (end 146.9963 72.7132) (width 0.25) (layer "F.Cu") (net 7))
 (segment (start 151.4502 59.148) (end 150.1962 59.148) (width 0.25) (layer "F.Cu") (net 7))
 (segment (start 150.1962 59.6338) (end 147.6 62.23) (width 0.25) (layer "F.Cu") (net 7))
 (segment (start 146.9963 62.8337) (end 147.6 62.23) (width 0.25) (layer "F.Cu") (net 7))
 (segment (start 146.9963 72.7132) (end 146.9963 62.8337) (width 0.25) (layer "F.Cu") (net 7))
 (segment (start 150.1962 59.148) (end 150.1962 59.6338) (width 0.25) (layer "F.Cu") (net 7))
 (segment (start 149.86 73.66) (end 147.9431 73.66) (width 0.25) (layer "F.Cu") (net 7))
 (segment (start 149.86 68.58) (end 151.7769 68.58) (width 0.25) (layer "F.Cu") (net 5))
 (segment (start 158.367 63.6151) (end 158.1652 63.6151) (width 0.25) (layer "F.Cu") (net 5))
 (segment (start 156.9112 62.958) (end 158.1652 62.958) (width 0.25) (layer "F.Cu") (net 5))
 (segment (start 158.1652 63.6151) (end 156.7418 63.6151) (width 0.25) (layer "F.Cu") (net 5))
 (segment (start 156.7418 63.6151) (end 151.7769 68.58) (width 0.25) (layer "F.Cu") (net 5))
 (segment (start 162.37 68.58) (end 162.37 67.6181) (width 0.25) (layer "F.Cu") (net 5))
 (segment (start 162.37 67.6181) (end 158.367 63.6151) (width 0.25) (layer "F.Cu") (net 5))
 (segment (start 158.1652 63.6151) (end 158.1652 62.958) (width 0.25) (layer "F.Cu") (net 5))
 (segment (start 152.4412 72.0819) (end 148.108 72.0819) (width 0.25) (layer "F.Cu") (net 8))
 (segment (start 148.108 72.0819) (end 147.4868 71.4607) (width 0.25) (layer "F.Cu") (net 8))
 (segment (start 155.32 71.12) (end 153.4031 71.12) (width 0.25) (layer "F.Cu") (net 8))
 (segment (start 151.4502 62.958) (end 150.1962 62.958) (width 0.25) (layer "F.Cu") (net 8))
 (segment (start 153.4031 71.12) (end 152.4412 72.0819) (width 0.25) (layer "F.Cu") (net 8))
 (segment (start 147.4868 71.4607) (end 147.4868 65.6674) (width 0.25) (layer "F.Cu") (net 8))
 (segment (start 147.4868 65.6674) (end 150.1962 62.958) (width 0.25) (layer "F.Cu") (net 8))
 (segment (start 156.9112 61.688) (end 155.6572 61.688) (width 0.25) (layer "F.Cu") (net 6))
 (segment (start 155.6572 61.688) (end 151.9546 65.3906) (width 0.25) (layer "F.Cu") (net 6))
 (segment (start 149.86 71.12) (end 147.9431 71.12) (width 0.25) (layer "F.Cu") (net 6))
 (segment (start 151.9546 65.3906) (end 150.2981 65.3906) (width 0.25) (layer "F.Cu") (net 6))
 (segment (start 147.9431 67.7456) (end 147.9431 71.12) (width 0.25) (layer "F.Cu") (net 6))
 (segment (start 150.2981 65.3906) (end 147.9431 67.7456) (width 0.25) (layer "F.Cu") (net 6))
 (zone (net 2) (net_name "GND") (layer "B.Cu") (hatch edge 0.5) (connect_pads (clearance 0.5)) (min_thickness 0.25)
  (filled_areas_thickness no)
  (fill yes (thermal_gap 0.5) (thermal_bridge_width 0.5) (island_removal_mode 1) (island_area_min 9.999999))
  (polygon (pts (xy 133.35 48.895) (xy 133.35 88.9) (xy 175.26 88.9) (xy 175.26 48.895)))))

